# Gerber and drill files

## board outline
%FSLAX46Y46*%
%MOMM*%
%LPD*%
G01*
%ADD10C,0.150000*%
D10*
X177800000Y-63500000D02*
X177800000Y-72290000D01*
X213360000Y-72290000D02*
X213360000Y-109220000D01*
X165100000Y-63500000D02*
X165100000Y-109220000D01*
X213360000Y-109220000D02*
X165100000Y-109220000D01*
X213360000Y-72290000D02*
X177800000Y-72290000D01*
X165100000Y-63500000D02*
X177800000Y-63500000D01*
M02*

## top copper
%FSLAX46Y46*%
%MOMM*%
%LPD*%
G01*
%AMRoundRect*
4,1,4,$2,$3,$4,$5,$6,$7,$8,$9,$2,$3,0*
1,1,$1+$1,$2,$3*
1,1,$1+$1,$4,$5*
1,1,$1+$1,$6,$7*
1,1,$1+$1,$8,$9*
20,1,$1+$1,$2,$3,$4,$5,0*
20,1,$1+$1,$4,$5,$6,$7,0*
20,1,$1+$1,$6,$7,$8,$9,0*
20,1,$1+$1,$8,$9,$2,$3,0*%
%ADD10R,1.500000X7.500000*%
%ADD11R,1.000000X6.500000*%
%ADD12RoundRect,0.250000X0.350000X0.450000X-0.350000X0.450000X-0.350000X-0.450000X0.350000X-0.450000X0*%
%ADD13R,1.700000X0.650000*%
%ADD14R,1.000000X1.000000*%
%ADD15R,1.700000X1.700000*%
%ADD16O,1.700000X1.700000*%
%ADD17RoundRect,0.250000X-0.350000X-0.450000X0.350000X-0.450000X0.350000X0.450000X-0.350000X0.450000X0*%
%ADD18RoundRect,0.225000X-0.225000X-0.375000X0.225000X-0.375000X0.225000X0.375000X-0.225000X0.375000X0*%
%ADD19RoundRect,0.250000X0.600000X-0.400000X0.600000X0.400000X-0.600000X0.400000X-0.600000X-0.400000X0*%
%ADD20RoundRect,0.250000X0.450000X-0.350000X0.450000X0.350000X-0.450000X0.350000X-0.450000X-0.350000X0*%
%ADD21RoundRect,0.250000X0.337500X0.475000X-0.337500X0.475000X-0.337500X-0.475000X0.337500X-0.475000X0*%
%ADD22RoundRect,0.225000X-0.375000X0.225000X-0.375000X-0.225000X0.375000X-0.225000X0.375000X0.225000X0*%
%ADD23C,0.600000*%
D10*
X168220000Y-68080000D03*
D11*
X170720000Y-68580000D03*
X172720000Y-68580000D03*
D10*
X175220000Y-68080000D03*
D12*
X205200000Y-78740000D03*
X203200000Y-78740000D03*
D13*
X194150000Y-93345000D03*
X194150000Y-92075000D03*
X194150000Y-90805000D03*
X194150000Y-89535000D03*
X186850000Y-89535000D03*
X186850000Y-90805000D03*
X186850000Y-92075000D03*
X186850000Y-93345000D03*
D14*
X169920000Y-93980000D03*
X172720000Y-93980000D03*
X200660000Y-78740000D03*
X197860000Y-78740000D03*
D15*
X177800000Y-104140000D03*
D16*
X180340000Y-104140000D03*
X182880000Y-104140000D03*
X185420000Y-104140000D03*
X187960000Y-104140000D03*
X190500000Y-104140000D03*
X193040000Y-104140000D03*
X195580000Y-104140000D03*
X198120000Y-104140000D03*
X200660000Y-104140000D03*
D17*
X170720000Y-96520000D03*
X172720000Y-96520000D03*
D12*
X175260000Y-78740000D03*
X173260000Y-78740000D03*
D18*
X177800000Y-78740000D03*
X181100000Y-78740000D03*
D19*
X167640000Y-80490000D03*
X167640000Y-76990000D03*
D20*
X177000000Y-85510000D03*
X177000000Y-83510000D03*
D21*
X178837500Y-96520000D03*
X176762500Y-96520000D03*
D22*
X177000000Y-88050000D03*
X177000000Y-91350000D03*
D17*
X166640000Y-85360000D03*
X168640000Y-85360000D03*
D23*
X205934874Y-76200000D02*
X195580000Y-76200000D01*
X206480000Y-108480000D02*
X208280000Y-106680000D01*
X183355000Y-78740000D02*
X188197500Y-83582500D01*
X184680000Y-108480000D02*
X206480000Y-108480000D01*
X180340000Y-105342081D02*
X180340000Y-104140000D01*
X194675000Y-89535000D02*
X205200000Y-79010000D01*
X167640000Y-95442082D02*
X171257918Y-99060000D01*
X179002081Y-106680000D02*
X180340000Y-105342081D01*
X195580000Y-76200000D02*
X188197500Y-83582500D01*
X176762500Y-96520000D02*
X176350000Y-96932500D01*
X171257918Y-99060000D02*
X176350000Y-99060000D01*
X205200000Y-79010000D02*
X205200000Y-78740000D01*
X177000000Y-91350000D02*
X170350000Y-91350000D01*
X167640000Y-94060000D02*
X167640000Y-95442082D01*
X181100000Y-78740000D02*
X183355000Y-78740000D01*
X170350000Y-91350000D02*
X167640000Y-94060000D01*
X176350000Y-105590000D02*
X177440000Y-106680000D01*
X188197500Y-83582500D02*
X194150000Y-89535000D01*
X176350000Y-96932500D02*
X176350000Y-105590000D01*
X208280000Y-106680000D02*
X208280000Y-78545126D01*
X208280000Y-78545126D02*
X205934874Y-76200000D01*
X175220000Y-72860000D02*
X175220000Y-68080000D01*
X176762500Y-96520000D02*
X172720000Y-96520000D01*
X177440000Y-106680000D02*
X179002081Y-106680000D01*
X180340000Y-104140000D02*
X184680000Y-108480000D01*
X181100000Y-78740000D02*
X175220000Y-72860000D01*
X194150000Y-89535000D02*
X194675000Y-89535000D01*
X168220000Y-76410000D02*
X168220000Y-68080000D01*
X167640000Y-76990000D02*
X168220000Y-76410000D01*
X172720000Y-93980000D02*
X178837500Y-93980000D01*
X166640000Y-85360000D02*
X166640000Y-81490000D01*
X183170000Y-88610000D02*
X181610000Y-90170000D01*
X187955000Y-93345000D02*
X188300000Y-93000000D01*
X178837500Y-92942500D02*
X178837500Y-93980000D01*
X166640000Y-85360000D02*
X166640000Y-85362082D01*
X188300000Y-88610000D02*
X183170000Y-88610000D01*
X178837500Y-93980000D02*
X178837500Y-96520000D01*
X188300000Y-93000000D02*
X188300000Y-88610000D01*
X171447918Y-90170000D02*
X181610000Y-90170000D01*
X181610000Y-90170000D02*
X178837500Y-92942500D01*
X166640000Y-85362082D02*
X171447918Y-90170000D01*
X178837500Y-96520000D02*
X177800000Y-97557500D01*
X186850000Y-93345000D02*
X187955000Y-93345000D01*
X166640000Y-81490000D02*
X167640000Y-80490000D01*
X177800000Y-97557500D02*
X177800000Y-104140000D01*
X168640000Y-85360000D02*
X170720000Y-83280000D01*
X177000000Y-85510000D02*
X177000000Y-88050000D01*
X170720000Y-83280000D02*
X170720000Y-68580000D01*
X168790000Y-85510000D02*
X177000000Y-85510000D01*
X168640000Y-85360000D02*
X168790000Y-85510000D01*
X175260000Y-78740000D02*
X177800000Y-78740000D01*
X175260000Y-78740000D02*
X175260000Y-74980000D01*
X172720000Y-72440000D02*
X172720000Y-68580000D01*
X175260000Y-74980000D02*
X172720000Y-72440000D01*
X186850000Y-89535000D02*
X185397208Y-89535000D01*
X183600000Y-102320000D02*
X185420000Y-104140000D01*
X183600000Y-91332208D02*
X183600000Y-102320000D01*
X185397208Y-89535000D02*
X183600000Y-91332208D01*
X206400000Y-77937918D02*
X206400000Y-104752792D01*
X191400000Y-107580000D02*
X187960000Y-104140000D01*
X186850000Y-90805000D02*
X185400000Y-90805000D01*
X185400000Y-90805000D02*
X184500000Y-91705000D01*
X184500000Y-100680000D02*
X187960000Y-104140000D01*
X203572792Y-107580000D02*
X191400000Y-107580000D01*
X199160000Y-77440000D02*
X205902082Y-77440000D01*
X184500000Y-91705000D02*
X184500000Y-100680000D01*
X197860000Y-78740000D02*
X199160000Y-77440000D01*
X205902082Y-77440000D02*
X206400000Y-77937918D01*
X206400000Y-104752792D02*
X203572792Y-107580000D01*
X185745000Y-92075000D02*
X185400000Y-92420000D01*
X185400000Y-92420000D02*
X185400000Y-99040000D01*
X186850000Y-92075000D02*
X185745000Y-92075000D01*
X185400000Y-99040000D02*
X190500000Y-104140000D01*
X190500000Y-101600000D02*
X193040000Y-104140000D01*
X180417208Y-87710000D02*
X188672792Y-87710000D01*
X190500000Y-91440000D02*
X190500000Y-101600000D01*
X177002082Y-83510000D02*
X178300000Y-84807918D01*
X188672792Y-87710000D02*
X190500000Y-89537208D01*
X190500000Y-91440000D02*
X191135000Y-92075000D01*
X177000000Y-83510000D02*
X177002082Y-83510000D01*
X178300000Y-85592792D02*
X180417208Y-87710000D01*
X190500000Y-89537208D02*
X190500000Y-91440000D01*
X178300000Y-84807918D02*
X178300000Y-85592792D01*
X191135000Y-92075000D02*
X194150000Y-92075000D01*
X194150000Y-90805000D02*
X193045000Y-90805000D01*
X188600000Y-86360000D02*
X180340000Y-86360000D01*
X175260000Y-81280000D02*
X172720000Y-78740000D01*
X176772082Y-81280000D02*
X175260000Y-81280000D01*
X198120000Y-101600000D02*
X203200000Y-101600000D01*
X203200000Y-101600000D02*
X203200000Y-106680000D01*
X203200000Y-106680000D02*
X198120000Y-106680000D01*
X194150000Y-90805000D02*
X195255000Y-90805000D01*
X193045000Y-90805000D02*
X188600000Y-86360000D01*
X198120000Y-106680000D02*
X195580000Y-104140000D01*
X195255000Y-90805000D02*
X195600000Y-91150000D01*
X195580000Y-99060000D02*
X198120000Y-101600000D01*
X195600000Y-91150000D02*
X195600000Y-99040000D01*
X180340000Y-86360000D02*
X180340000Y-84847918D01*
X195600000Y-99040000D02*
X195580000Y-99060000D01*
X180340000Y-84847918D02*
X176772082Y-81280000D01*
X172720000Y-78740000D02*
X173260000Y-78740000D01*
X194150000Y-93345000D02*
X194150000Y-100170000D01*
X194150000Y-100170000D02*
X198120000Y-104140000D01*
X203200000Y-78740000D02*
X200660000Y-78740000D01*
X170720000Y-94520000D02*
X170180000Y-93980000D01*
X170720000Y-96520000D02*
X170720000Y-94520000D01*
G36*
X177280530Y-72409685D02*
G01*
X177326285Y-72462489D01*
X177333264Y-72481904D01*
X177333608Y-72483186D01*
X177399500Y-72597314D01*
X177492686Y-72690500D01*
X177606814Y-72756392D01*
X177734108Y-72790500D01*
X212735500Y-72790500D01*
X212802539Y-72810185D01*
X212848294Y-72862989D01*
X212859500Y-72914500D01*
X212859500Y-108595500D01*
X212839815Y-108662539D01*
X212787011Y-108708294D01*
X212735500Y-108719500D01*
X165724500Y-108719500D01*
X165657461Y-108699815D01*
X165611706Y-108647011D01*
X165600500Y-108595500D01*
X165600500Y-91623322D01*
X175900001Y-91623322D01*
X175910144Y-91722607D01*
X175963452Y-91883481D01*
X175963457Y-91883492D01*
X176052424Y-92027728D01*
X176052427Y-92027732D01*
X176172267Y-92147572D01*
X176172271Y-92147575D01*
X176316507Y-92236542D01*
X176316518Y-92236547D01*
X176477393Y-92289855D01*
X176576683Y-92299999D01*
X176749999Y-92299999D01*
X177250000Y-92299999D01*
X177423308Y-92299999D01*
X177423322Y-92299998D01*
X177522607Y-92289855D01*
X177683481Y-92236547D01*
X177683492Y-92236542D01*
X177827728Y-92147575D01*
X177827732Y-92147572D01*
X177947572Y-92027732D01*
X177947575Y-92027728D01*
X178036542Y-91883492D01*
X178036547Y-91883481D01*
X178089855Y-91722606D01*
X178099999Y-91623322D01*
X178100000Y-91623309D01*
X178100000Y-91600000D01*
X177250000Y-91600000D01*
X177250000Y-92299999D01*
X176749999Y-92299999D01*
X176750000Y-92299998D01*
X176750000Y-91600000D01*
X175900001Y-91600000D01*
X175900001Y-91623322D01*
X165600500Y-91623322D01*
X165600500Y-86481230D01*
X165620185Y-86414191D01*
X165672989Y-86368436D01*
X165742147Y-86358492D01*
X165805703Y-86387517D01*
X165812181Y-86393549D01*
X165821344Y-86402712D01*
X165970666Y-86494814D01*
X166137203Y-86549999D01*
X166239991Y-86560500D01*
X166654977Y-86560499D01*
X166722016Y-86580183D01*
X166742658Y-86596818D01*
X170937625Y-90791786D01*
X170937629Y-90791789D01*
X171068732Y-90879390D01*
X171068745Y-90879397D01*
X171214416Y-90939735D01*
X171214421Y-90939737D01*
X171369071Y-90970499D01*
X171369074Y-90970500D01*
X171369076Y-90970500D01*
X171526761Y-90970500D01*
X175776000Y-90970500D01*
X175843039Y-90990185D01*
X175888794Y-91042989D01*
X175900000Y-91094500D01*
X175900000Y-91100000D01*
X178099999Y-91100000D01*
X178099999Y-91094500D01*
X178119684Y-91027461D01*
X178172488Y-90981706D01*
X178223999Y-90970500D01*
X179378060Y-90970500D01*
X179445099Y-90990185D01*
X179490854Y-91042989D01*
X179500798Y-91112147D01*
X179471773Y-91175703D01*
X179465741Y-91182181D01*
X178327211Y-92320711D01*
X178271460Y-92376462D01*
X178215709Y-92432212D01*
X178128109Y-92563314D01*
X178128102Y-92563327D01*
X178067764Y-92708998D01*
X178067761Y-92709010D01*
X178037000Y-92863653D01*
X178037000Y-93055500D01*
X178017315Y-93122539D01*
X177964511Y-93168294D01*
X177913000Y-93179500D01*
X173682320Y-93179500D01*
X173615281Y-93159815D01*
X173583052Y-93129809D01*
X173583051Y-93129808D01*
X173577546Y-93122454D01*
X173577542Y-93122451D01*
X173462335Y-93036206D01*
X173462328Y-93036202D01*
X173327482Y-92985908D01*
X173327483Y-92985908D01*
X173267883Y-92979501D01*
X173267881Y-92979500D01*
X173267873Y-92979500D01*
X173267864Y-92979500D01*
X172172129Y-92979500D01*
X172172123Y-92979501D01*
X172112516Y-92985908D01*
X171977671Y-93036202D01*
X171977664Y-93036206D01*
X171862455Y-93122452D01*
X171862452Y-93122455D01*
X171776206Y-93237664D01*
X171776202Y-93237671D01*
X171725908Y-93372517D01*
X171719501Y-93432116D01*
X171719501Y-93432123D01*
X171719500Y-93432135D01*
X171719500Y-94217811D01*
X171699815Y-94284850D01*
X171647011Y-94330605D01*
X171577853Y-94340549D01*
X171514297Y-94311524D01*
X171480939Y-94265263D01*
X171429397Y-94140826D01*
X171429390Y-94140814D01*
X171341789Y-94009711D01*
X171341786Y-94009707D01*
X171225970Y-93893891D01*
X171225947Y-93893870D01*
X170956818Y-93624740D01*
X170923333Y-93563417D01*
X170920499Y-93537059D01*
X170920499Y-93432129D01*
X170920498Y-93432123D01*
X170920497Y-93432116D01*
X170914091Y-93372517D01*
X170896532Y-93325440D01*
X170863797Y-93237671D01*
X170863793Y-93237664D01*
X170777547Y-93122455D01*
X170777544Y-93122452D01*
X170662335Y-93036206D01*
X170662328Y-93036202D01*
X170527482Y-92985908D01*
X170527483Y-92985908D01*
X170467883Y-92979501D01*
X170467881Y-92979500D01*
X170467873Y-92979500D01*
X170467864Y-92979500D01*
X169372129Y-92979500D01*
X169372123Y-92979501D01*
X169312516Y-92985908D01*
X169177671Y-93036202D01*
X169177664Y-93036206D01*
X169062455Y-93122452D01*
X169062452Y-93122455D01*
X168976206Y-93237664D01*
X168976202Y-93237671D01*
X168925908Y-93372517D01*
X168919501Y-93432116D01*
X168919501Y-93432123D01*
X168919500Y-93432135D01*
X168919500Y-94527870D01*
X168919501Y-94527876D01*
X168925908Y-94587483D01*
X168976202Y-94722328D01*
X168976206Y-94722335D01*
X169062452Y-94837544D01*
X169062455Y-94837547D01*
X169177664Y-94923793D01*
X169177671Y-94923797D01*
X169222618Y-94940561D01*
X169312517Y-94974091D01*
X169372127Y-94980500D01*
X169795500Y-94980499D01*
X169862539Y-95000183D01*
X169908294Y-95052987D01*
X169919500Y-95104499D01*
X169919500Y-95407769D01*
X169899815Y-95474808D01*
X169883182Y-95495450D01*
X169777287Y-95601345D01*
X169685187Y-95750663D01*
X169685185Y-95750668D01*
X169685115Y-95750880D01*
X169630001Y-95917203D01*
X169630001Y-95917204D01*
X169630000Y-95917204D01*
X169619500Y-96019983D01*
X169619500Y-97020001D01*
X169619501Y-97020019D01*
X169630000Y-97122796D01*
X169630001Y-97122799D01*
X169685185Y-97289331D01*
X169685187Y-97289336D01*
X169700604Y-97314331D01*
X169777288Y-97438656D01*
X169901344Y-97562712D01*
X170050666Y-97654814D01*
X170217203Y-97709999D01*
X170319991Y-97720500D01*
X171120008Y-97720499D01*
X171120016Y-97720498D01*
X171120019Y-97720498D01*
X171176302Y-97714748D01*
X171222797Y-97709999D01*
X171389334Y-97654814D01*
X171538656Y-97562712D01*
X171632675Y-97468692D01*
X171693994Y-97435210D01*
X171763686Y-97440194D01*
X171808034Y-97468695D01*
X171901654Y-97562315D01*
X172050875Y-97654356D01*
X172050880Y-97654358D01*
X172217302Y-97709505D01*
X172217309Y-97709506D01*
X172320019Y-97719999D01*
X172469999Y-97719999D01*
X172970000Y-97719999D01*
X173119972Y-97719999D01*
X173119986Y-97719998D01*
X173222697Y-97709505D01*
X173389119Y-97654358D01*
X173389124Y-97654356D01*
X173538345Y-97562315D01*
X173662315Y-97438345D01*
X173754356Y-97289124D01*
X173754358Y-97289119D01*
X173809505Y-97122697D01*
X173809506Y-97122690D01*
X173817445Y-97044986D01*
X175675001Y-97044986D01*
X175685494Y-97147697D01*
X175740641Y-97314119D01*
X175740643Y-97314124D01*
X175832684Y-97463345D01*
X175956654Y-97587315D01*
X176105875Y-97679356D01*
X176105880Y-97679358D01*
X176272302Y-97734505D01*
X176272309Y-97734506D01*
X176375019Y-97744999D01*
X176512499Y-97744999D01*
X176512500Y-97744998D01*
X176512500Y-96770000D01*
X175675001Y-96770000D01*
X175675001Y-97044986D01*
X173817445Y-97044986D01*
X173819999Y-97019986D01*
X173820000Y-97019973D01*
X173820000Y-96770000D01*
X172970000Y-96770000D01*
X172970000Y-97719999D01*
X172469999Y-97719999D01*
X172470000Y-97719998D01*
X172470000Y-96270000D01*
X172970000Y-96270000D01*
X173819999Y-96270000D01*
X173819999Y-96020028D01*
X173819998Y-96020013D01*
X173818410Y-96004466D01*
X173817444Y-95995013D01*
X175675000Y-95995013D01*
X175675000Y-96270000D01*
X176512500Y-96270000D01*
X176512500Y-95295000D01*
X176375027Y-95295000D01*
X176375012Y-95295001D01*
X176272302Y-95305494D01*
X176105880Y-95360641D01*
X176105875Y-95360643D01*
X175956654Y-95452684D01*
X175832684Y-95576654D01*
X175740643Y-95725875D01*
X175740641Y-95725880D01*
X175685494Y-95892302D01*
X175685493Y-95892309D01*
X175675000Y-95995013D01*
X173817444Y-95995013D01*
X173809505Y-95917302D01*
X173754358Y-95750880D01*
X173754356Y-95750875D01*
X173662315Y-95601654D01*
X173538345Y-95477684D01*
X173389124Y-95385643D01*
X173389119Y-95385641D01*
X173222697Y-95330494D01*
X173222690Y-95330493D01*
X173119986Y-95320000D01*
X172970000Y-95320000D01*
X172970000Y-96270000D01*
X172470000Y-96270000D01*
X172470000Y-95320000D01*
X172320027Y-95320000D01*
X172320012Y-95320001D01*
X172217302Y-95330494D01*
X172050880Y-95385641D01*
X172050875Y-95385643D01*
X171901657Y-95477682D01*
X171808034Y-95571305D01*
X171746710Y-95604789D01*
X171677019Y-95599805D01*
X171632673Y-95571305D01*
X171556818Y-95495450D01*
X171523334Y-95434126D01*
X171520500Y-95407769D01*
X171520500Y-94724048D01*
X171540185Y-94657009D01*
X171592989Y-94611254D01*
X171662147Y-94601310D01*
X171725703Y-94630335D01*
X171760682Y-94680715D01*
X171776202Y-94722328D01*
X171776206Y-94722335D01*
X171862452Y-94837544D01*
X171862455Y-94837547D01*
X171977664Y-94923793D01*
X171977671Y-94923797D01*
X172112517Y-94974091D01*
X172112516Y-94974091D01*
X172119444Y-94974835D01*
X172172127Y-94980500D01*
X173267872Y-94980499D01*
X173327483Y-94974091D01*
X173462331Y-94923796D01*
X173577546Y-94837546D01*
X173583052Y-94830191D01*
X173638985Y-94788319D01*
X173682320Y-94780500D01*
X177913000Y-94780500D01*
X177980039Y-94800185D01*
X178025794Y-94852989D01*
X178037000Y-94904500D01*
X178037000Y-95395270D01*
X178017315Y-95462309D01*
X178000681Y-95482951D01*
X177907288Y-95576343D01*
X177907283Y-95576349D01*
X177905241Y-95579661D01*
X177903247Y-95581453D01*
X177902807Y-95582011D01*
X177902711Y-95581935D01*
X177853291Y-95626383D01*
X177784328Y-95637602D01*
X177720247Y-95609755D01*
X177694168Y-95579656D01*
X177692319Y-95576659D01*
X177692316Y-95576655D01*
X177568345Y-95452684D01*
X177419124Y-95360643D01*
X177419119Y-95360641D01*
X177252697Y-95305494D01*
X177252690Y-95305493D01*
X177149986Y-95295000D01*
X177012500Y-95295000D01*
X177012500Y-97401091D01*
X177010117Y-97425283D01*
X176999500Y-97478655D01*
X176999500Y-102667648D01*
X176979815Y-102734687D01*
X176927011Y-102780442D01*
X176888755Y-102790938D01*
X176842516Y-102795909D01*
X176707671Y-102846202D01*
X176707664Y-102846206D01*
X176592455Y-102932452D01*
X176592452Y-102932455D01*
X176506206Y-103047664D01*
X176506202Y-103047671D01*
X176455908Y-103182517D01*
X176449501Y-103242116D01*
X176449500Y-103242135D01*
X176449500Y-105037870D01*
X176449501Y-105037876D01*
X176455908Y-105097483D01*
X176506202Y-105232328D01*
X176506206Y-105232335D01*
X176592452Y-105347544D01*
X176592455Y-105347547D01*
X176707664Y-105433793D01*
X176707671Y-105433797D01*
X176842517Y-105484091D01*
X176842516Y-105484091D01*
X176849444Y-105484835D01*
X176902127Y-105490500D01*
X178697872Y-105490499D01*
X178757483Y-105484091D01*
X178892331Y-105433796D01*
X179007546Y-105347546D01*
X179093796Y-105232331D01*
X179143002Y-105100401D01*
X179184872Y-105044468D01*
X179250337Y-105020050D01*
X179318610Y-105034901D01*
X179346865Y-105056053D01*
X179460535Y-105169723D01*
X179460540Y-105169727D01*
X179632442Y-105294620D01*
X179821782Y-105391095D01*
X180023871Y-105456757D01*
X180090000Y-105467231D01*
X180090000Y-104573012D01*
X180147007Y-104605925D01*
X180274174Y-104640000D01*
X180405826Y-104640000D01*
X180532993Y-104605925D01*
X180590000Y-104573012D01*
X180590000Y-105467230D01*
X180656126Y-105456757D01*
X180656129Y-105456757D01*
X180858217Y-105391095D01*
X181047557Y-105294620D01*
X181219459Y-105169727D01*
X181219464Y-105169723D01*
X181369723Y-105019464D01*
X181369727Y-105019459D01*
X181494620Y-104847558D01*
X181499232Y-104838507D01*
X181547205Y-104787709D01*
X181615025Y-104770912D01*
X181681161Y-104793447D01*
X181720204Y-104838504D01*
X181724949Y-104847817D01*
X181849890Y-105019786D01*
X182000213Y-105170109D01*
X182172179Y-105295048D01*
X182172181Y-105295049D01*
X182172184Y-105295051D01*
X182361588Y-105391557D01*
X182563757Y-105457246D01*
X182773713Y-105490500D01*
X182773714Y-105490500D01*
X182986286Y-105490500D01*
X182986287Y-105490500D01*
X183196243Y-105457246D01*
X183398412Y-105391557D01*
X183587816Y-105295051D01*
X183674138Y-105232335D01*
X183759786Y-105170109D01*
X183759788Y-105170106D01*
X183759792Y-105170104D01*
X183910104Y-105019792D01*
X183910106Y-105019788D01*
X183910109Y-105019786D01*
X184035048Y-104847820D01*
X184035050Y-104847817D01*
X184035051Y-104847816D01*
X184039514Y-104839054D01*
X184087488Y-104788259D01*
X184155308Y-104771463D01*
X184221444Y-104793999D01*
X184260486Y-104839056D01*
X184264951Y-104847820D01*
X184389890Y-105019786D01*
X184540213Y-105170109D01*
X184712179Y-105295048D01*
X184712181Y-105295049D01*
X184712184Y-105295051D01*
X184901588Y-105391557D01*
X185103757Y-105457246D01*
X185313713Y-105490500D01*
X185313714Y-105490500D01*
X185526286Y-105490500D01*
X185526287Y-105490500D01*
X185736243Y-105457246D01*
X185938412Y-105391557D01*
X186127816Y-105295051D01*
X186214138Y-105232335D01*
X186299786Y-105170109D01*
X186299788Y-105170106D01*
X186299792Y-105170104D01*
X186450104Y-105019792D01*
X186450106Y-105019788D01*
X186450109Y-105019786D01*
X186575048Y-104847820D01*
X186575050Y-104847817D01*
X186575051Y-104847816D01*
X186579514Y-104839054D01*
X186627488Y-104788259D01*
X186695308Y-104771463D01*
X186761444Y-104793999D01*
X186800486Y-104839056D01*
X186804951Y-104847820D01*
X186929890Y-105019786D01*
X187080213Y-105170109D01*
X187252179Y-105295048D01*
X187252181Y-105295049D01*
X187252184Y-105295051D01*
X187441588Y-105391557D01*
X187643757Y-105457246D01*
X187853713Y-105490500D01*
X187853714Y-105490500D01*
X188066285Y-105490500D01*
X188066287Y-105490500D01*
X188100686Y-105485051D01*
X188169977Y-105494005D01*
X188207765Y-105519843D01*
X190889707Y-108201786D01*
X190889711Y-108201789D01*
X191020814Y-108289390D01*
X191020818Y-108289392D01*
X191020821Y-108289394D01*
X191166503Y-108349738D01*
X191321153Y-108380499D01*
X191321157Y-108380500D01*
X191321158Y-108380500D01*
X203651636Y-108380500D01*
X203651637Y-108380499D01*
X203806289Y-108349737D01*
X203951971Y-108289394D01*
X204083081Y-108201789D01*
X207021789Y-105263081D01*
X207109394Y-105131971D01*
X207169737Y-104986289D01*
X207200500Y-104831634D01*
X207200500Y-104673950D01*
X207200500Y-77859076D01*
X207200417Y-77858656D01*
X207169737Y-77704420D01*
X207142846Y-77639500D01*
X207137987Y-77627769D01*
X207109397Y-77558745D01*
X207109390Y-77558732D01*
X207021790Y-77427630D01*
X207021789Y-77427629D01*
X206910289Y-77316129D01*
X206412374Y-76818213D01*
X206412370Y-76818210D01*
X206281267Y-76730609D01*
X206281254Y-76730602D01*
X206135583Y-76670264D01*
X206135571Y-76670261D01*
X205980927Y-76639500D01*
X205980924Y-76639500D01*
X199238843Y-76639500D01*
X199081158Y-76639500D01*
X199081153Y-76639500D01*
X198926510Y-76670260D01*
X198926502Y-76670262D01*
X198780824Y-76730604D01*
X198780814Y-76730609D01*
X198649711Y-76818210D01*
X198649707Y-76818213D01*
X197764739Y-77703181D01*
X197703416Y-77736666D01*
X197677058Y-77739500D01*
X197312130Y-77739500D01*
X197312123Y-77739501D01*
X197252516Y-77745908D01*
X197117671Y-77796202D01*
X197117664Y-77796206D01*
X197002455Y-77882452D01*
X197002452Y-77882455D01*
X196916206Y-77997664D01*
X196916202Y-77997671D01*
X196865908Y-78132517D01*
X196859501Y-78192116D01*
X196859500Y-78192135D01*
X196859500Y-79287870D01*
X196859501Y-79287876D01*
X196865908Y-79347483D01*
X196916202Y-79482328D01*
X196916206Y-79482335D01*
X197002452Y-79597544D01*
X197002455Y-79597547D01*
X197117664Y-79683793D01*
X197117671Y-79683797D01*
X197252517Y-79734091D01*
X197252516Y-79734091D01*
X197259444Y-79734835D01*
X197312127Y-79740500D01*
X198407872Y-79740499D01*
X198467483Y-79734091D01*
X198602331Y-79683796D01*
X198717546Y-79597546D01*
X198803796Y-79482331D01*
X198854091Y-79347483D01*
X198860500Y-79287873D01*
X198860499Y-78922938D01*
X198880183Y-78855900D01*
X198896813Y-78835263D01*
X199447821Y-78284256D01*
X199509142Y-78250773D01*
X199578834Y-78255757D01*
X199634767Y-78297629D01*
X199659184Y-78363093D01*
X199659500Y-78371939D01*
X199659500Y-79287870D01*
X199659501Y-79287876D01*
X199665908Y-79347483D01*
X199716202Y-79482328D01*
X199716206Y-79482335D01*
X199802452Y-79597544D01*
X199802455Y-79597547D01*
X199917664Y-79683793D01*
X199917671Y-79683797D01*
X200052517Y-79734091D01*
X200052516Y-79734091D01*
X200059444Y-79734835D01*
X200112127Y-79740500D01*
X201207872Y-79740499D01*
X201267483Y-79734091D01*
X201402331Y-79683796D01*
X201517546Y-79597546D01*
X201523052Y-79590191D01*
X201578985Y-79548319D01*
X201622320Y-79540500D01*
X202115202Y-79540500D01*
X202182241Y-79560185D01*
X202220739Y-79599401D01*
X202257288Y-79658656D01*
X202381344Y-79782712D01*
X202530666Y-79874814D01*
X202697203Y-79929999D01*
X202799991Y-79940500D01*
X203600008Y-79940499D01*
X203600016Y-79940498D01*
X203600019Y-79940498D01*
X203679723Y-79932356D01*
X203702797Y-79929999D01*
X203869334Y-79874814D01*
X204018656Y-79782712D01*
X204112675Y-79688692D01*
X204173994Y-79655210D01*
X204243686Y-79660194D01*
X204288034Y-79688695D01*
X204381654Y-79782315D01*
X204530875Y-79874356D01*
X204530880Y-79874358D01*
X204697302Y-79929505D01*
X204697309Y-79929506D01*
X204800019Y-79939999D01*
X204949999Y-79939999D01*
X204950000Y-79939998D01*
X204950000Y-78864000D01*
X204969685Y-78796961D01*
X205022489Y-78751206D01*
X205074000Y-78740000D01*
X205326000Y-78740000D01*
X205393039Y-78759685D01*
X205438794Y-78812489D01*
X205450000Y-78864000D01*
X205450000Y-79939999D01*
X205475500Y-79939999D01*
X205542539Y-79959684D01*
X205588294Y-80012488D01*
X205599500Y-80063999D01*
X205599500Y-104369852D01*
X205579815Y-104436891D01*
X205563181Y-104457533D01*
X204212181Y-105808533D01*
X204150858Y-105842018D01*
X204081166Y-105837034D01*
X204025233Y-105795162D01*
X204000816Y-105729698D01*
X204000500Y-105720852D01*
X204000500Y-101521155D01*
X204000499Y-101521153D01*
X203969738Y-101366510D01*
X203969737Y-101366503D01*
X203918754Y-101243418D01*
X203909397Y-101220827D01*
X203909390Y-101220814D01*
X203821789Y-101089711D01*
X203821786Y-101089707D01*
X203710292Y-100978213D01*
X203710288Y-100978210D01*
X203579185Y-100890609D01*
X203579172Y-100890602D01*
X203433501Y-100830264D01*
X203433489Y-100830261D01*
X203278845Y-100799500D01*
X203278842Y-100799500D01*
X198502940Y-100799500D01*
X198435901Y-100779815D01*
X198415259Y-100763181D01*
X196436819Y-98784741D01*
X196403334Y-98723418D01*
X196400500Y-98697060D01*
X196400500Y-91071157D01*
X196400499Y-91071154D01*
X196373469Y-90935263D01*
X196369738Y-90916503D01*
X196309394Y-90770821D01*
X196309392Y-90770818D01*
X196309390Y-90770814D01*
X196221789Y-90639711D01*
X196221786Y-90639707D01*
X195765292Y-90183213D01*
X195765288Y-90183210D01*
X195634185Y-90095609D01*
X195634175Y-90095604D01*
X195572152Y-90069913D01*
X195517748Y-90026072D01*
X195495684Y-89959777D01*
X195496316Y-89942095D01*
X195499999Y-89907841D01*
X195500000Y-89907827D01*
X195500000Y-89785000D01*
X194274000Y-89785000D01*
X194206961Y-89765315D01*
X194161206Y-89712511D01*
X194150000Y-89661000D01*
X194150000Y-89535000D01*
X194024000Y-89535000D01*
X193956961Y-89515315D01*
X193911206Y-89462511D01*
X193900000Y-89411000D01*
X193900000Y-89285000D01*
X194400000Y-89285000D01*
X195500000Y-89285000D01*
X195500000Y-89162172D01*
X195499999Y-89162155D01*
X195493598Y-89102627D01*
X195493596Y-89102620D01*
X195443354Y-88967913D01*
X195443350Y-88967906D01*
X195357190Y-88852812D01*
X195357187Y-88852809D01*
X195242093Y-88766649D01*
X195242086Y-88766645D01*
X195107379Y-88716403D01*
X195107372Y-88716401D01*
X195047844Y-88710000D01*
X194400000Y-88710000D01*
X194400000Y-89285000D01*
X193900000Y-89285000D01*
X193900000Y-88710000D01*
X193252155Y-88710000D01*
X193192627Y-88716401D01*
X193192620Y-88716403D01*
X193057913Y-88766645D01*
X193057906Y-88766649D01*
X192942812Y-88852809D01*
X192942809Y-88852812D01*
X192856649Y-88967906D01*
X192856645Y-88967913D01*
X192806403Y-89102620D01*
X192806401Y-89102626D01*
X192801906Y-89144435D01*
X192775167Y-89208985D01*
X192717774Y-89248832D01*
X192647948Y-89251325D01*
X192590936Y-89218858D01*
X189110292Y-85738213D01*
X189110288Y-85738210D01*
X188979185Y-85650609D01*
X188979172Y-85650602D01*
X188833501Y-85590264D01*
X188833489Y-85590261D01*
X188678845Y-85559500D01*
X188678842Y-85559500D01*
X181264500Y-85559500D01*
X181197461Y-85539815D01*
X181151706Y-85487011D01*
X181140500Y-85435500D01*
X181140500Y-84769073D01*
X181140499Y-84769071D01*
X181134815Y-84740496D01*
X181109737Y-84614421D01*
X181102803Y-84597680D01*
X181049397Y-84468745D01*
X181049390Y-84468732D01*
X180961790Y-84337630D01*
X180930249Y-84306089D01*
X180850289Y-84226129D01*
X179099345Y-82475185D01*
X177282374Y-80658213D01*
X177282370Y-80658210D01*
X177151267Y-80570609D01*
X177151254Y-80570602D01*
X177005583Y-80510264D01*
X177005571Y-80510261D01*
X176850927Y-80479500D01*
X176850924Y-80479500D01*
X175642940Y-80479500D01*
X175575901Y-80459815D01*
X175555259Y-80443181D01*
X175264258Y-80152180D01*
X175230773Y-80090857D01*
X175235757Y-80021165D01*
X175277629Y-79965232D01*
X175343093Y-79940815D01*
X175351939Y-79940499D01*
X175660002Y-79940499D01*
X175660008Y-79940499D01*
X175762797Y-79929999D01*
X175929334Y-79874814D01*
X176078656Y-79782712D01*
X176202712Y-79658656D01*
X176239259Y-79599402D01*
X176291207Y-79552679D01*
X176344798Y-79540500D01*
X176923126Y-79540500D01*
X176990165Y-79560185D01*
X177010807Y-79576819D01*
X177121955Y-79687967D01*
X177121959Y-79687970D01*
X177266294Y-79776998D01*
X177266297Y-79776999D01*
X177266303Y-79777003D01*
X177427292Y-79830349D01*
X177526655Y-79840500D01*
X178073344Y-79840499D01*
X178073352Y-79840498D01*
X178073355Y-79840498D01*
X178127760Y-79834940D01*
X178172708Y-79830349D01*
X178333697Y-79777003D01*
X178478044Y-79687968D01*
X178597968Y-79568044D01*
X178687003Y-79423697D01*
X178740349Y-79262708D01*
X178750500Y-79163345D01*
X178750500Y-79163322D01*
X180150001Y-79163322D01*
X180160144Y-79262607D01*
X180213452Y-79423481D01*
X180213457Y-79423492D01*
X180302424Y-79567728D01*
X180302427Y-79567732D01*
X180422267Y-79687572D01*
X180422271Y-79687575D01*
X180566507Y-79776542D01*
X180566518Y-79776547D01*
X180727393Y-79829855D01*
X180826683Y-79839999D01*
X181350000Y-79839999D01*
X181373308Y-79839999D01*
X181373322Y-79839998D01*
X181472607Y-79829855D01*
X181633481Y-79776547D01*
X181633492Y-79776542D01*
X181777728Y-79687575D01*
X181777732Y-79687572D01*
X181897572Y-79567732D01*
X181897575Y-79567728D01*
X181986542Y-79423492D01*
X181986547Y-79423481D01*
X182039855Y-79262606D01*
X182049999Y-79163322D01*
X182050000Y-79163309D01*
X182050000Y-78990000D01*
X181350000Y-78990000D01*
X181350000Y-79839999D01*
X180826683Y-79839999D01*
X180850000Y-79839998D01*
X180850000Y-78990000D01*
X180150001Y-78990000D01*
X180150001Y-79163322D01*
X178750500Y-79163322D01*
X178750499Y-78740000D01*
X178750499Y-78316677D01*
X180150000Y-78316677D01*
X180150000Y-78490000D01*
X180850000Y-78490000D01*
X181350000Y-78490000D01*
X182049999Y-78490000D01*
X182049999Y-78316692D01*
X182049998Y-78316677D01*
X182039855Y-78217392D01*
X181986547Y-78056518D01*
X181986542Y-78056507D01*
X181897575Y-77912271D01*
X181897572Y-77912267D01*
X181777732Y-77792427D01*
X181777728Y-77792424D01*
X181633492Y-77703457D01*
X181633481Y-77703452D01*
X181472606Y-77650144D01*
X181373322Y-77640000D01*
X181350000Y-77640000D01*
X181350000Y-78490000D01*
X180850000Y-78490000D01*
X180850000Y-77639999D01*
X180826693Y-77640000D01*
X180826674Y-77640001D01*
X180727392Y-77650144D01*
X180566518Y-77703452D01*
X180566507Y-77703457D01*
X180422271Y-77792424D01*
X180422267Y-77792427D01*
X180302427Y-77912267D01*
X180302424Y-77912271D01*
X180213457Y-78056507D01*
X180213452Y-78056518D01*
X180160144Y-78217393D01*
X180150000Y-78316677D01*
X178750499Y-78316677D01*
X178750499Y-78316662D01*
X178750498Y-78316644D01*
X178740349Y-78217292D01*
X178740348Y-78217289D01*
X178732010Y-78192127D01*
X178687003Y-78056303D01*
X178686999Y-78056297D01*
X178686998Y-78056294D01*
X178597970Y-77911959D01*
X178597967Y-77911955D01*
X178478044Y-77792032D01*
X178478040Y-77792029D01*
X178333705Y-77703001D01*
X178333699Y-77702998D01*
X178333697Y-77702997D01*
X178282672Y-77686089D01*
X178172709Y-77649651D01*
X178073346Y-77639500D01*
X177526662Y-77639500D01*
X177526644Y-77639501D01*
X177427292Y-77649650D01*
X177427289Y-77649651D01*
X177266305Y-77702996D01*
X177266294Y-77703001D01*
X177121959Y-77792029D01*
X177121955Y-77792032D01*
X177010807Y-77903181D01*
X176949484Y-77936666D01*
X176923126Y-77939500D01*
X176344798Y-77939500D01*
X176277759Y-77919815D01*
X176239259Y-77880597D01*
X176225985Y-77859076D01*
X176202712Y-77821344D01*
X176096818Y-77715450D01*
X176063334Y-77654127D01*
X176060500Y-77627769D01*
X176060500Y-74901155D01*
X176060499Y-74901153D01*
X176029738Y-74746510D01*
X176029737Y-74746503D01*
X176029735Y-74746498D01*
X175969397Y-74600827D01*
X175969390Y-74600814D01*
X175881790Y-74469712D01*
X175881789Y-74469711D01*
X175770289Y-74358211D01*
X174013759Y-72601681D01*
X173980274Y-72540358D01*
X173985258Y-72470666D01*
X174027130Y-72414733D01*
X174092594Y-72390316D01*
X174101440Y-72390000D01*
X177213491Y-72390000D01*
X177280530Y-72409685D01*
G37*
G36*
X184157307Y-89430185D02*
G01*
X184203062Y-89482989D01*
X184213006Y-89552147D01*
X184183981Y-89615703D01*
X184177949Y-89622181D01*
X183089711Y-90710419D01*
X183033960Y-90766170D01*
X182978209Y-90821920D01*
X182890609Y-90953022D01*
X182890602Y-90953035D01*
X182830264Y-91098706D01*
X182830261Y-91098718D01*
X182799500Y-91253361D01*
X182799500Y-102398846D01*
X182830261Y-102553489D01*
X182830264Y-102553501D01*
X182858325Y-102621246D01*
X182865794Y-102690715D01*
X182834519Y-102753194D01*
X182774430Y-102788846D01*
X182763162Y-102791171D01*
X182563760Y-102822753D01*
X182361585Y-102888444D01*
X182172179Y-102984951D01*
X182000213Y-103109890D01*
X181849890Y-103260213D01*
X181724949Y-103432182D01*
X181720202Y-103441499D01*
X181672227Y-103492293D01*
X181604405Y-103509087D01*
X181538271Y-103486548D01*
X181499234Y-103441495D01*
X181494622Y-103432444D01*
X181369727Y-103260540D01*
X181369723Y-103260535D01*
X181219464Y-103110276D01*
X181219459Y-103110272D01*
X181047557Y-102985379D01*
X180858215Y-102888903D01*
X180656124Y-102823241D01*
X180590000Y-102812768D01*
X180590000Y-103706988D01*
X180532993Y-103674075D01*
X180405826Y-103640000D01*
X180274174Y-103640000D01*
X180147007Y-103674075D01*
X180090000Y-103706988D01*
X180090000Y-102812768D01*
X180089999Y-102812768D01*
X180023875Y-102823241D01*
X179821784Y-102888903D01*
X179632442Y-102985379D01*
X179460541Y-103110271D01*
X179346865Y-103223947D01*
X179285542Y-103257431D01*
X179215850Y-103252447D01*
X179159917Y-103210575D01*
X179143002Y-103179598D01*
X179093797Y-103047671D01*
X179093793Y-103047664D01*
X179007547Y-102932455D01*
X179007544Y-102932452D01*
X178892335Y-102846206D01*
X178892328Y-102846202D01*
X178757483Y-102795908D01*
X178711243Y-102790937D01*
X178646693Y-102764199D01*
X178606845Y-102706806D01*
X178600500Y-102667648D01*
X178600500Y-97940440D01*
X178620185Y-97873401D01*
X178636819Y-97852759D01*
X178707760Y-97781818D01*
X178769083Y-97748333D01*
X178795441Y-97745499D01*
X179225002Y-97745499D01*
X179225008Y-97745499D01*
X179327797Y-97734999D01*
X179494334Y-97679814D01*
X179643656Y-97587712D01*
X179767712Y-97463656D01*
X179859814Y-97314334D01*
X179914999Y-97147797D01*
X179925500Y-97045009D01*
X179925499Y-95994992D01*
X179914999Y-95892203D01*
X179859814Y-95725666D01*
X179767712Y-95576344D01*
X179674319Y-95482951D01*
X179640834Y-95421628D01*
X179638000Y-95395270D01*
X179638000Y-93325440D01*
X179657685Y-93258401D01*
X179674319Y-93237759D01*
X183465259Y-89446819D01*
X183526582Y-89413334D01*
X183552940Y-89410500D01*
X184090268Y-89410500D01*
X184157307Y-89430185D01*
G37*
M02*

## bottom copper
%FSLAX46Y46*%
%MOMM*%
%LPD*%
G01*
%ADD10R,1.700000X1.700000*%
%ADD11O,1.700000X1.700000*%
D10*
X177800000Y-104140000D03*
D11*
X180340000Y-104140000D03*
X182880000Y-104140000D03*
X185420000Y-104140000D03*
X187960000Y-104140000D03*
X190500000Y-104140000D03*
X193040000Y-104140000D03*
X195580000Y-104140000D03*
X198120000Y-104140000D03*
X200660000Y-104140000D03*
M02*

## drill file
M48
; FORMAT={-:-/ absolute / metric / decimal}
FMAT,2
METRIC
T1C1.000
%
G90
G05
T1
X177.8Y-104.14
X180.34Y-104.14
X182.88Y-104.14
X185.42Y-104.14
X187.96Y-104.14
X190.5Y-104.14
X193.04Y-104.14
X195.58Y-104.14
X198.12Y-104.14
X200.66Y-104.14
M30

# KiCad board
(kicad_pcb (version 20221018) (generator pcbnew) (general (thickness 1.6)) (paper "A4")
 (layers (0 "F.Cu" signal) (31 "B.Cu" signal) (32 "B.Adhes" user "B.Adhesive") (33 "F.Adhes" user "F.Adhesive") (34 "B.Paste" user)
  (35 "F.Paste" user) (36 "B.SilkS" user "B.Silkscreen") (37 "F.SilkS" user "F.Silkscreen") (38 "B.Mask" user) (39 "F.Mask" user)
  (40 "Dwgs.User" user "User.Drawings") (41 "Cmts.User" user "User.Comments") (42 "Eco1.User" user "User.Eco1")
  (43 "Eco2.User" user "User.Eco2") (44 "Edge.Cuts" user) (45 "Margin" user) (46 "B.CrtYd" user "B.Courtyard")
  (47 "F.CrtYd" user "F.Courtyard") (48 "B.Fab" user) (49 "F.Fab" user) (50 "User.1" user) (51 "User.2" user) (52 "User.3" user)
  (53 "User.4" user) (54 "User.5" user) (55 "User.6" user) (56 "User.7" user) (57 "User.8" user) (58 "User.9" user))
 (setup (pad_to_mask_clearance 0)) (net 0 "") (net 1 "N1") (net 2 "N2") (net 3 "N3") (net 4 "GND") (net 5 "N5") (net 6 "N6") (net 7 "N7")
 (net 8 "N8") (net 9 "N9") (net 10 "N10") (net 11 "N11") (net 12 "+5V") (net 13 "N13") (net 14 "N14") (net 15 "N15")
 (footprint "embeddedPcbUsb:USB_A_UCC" (layer "F.Cu") (at 171.72 68.28 -90)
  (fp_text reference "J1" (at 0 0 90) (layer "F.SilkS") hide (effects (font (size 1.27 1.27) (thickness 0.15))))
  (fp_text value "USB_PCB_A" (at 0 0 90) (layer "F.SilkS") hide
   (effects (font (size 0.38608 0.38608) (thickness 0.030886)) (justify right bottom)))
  (pad "1" smd rect (at -0.2 3.5 270) (size 7.5 1.5) (layers "F.Cu" "F.Paste" "F.Mask") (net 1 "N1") (solder_mask_margin 0.1016))
  (pad "2" smd rect (at 0.3 1 270) (size 6.5 1) (layers "F.Cu" "F.Paste" "F.Mask") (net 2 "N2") (solder_mask_margin 0.1016))
  (pad "3" smd rect (at 0.3 -1 270) (size 6.5 1) (layers "F.Cu" "F.Paste" "F.Mask") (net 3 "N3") (solder_mask_margin 0.1016))
  (pad "4" smd rect (at -0.2 -3.5 270) (size 7.5 1.5) (layers "F.Cu" "F.Paste" "F.Mask") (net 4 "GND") (solder_mask_margin 0.1016)))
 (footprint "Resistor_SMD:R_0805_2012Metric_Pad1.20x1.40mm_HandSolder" (layer "F.Cu") (at 204.2 78.74 180)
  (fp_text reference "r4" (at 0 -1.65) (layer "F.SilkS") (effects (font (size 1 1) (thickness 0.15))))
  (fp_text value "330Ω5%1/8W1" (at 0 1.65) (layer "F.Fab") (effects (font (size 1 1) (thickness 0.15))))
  (pad "1" smd roundrect (at -1 0 180) (size 1.2 1.4) (layers "F.Cu" "F.Paste" "F.Mask") (roundrect_rratio 0.208333) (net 4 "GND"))
  (pad "2" smd roundrect (at 1 0 180) (size 1.2 1.4) (layers "F.Cu" "F.Paste" "F.Mask") (roundrect_rratio 0.208333) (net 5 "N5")))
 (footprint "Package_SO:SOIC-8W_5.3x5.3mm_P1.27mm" (layer "F.Cu") (at 190.5 91.44 180)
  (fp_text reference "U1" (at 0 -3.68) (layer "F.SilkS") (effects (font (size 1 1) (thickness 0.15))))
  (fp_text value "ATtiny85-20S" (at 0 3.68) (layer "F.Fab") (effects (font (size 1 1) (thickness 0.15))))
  (pad "1" smd rect (at -3.65 -1.905 180) (size 1.7 0.65) (layers "F.Cu" "F.Paste" "F.Mask") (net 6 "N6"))
  (pad "2" smd rect (at -3.65 -0.635 180) (size 1.7 0.65) (layers "F.Cu" "F.Paste" "F.Mask") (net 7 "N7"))
  (pad "3" smd rect (at -3.65 0.635 180) (size 1.7 0.65) (layers "F.Cu" "F.Paste" "F.Mask") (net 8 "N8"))
  (pad "4" smd rect (at -3.65 1.905 180) (size 1.7 0.65) (layers "F.Cu" "F.Paste" "F.Mask") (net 4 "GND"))
  (pad "5" smd rect (at 3.65 1.905 180) (size 1.7 0.65) (layers "F.Cu" "F.Paste" "F.Mask") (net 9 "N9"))
  (pad "6" smd rect (at 3.65 0.635 180) (size 1.7 0.65) (layers "F.Cu" "F.Paste" "F.Mask") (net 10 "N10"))
  (pad "7" smd rect (at 3.65 -0.635 180) (size 1.7 0.65) (layers "F.Cu" "F.Paste" "F.Mask") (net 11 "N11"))
  (pad "8" smd rect (at 3.65 -1.905 180) (size 1.7 0.65) (layers "F.Cu" "F.Paste" "F.Mask") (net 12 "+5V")))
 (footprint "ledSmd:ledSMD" (layer "F.Cu") (at 171.72 93.98)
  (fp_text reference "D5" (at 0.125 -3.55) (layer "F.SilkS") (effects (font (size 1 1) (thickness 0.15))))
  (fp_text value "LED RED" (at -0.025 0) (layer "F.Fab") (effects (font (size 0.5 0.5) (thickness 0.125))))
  (pad "1" smd rect (at -1.8 0) (size 1 1) (layers "F.Cu" "F.Paste" "F.Mask") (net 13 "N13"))
  (pad "2" smd rect (at 1 0) (size 1 1) (layers "F.Cu" "F.Paste" "F.Mask") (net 12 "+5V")))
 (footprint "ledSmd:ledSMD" (layer "F.Cu") (at 198.86 78.74 180)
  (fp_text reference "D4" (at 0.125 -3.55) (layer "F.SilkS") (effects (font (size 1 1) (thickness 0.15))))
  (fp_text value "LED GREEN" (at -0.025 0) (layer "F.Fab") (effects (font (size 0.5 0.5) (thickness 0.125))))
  (pad "1" smd rect (at -1.8 0 180) (size 1 1) (layers "F.Cu" "F.Paste" "F.Mask") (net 5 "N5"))
  (pad "2" smd rect (at 1 0 180) (size 1 1) (layers "F.Cu" "F.Paste" "F.Mask") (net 10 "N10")))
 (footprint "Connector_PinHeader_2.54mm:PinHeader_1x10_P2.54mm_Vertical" (layer "F.Cu") (at 177.8 104.14 90)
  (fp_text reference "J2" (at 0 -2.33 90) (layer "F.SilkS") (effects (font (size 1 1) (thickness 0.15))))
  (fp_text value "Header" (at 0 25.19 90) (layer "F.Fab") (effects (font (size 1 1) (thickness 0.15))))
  (pad "1" thru_hole rect (at 0 0 90) (size 1.7 1.7) (drill 1) (layers "*.Cu" "*.Mask") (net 12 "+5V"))
  (pad "2" thru_hole oval (at 0 2.54 90) (size 1.7 1.7) (drill 1) (layers "*.Cu" "*.Mask") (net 4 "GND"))
  (pad "3" thru_hole oval (at 0 5.08 90) (size 1.7 1.7) (drill 1) (layers "*.Cu" "*.Mask") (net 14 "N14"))
  (pad "4" thru_hole oval (at 0 7.62 90) (size 1.7 1.7) (drill 1) (layers "*.Cu" "*.Mask") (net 9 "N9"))
  (pad "5" thru_hole oval (at 0 10.16 90) (size 1.7 1.7) (drill 1) (layers "*.Cu" "*.Mask") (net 10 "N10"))
  (pad "6" thru_hole oval (at 0 12.7 90) (size 1.7 1.7) (drill 1) (layers "*.Cu" "*.Mask") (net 11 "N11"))
  (pad "7" thru_hole oval (at 0 15.24 90) (size 1.7 1.7) (drill 1) (layers "*.Cu" "*.Mask") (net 7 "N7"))
  (pad "8" thru_hole oval (at 0 17.78 90) (size 1.7 1.7) (drill 1) (layers "*.Cu" "*.Mask") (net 8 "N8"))
  (pad "9" thru_hole oval (at 0 20.32 90) (size 1.7 1.7) (drill 1) (layers "*.Cu" "*.Mask") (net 6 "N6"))
  (pad "10" thru_hole oval (at 0 22.86 90) (size 1.7 1.7) (drill 1) (layers "*.Cu" "*.Mask") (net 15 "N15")))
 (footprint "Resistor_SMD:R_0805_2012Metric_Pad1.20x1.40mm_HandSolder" (layer "F.Cu") (at 171.72 96.52)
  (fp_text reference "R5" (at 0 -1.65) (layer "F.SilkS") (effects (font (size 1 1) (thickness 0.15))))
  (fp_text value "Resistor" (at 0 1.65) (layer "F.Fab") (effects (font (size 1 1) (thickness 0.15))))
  (pad "1" smd roundrect (at -1 0) (size 1.2 1.4) (layers "F.Cu" "F.Paste" "F.Mask") (roundrect_rratio 0.208333) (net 13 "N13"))
  (pad "2" smd roundrect (at 1 0) (size 1.2 1.4) (layers "F.Cu" "F.Paste" "F.Mask") (roundrect_rratio 0.208333) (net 4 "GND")))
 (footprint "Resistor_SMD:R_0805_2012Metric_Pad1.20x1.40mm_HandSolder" (layer "F.Cu") (at 174.26 78.74 180)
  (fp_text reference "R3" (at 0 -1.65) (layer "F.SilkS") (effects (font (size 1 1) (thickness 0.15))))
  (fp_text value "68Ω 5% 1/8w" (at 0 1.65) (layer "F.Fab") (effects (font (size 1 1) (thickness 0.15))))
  (pad "1" smd roundrect (at -1 0 180) (size 1.2 1.4) (layers "F.Cu" "F.Paste" "F.Mask") (roundrect_rratio 0.208333) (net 3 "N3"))
  (pad "2" smd roundrect (at 1 0 180) (size 1.2 1.4) (layers "F.Cu" "F.Paste" "F.Mask") (roundrect_rratio 0.208333) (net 8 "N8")))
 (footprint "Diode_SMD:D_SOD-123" (layer "F.Cu") (at 179.45 78.74)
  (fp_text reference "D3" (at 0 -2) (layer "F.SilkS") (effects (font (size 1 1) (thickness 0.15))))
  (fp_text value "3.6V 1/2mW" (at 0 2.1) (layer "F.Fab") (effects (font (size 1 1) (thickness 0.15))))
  (pad "1" smd roundrect (at -1.65 0) (size 0.9 1.2) (layers "F.Cu" "F.Paste" "F.Mask") (roundrect_rratio 0.25) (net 3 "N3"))
  (pad "2" smd roundrect (at 1.65 0) (size 0.9 1.2) (layers "F.Cu" "F.Paste" "F.Mask") (roundrect_rratio 0.25) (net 4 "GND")))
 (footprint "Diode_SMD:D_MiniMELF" (layer "F.Cu") (at 167.64 78.74 90)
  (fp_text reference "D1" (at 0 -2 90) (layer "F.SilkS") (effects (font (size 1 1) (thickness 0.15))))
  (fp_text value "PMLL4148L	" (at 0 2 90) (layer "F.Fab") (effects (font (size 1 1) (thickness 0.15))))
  (pad "1" smd roundrect (at -1.75 0 90) (size 1.3 1.7) (layers "F.Cu" "F.Paste" "F.Mask") (roundrect_rratio 0.1923076923) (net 12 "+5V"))
  (pad "2" smd roundrect (at 1.75 0 90) (size 1.3 1.7) (layers "F.Cu" "F.Paste" "F.Mask") (roundrect_rratio 0.1923076923) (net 1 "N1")))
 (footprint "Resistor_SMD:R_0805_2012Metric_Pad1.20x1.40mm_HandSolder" (layer "F.Cu") (at 177 84.51 90)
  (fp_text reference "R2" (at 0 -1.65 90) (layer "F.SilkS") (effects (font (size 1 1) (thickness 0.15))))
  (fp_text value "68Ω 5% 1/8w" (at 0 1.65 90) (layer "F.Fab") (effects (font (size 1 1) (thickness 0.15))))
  (pad "1" smd roundrect (at -1 0 90) (size 1.2 1.4) (layers "F.Cu" "F.Paste" "F.Mask") (roundrect_rratio 0.208333) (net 2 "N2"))
  (pad "2" smd roundrect (at 1 0 90) (size 1.2 1.4) (layers "F.Cu" "F.Paste" "F.Mask") (roundrect_rratio 0.208333) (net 7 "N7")))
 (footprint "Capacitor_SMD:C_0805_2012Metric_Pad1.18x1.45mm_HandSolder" (layer "F.Cu") (at 177.8 96.52 180)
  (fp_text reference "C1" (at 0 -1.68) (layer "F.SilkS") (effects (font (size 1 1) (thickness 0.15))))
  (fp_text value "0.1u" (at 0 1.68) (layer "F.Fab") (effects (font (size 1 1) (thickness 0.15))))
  (pad "1" smd roundrect (at -1.0375 0 180) (size 1.175 1.45) (layers "F.Cu" "F.Paste" "F.Mask") (roundrect_rratio 0.212766) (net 12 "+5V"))
  (pad "2" smd roundrect (at 1.0375 0 180) (size 1.175 1.45) (layers "F.Cu" "F.Paste" "F.Mask") (roundrect_rratio 0.212766) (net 4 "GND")))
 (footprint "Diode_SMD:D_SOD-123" (layer "F.Cu") (at 177 89.7 -90)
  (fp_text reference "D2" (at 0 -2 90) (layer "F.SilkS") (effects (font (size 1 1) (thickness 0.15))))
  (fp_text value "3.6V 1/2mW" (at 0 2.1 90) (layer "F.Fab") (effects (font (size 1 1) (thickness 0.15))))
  (pad "1" smd roundrect (at -1.65 0 270) (size 0.9 1.2) (layers "F.Cu" "F.Paste" "F.Mask") (roundrect_rratio 0.25) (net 2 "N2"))
  (pad "2" smd roundrect (at 1.65 0 270) (size 0.9 1.2) (layers "F.Cu" "F.Paste" "F.Mask") (roundrect_rratio 0.25) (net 4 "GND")))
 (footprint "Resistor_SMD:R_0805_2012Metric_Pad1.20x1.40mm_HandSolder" (layer "F.Cu") (at 167.64 85.36)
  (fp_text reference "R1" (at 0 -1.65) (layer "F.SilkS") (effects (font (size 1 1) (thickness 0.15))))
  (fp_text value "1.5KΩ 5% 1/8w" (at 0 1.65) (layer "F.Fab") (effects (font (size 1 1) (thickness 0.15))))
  (pad "1" smd roundrect (at -1 0) (size 1.2 1.4) (layers "F.Cu" "F.Paste" "F.Mask") (roundrect_rratio 0.208333) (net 12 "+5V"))
  (pad "2" smd roundrect (at 1 0) (size 1.2 1.4) (layers "F.Cu" "F.Paste" "F.Mask") (roundrect_rratio 0.208333) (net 2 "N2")))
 (gr_line (start 177.8 63.5) (end 177.8 72.29) (stroke (width 0.15) (type default)) (layer "Edge.Cuts"))
 (gr_line (start 213.36 72.29) (end 213.36 109.22) (stroke (width 0.15) (type default)) (layer "Edge.Cuts"))
 (gr_line (start 165.1 63.5) (end 165.1 109.22) (stroke (width 0.15) (type default)) (layer "Edge.Cuts"))
 (gr_line (start 213.36 109.22) (end 165.1 109.22) (stroke (width 0.15) (type default)) (layer "Edge.Cuts"))
 (gr_line (start 213.36 72.29) (end 177.8 72.29) (stroke (width 0.15) (type default)) (layer "Edge.Cuts"))
 (gr_line (start 165.1 63.5) (end 177.8 63.5) (stroke (width 0.15) (type default)) (layer "Edge.Cuts"))
 (segment (start 205.934874 76.2) (end 195.58 76.2) (width 0.6) (layer "F.Cu") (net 4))
 (segment (start 206.48 108.48) (end 208.28 106.68) (width 0.6) (layer "F.Cu") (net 4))
 (segment (start 183.355 78.74) (end 188.1975 83.5825) (width 0.6) (layer "F.Cu") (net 4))
 (segment (start 184.68 108.48) (end 206.48 108.48) (width 0.6) (layer "F.Cu") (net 4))
 (segment (start 180.34 105.342081) (end 180.34 104.14) (width 0.6) (layer "F.Cu") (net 4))
 (segment (start 194.675 89.535) (end 205.2 79.01) (width 0.6) (layer "F.Cu") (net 4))
 (segment (start 167.64 95.442082) (end 171.257918 99.06) (width 0.6) (layer "F.Cu") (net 4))
 (segment (start 179.002081 106.68) (end 180.34 105.342081) (width 0.6) (layer "F.Cu") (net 4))
 (segment (start 195.58 76.2) (end 188.1975 83.5825) (width 0.6) (layer "F.Cu") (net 4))
 (segment (start 176.7625 96.52) (end 176.35 96.9325) (width 0.6) (layer "F.Cu") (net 4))
 (segment (start 171.257918 99.06) (end 176.35 99.06) (width 0.6) (layer "F.Cu") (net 4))
 (segment (start 205.2 79.01) (end 205.2 78.74) (width 0.6) (layer "F.Cu") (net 4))
 (segment (start 177 91.35) (end 170.35 91.35) (width 0.6) (layer "F.Cu") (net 4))
 (segment (start 167.64 94.06) (end 167.64 95.442082) (width 0.6) (layer "F.Cu") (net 4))
 (segment (start 181.1 78.74) (end 183.355 78.74) (width 0.6) (layer "F.Cu") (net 4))
 (segment (start 170.35 91.35) (end 167.64 94.06) (width 0.6) (layer "F.Cu") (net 4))
 (segment (start 176.35 105.59) (end 177.44 106.68) (width 0.6) (layer "F.Cu") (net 4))
 (segment (start 188.1975 83.5825) (end 194.15 89.535) (width 0.6) (layer "F.Cu") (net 4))
 (segment (start 176.35 96.9325) (end 176.35 105.59) (width 0.6) (layer "F.Cu") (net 4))
 (segment (start 208.28 106.68) (end 208.28 78.545126) (width 0.6) (layer "F.Cu") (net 4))
 (segment (start 208.28 78.545126) (end 205.934874 76.2) (width 0.6) (layer "F.Cu") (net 4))
 (segment (start 175.22 72.86) (end 175.22 68.08) (width 0.6) (layer "F.Cu") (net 4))
 (segment (start 176.7625 96.52) (end 172.72 96.52) (width 0.6) (layer "F.Cu") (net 4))
 (segment (start 177.44 106.68) (end 179.002081 106.68) (width 0.6) (layer "F.Cu") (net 4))
 (segment (start 180.34 104.14) (end 184.68 108.48) (width 0.6) (layer "F.Cu") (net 4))
 (segment (start 181.1 78.74) (end 175.22 72.86) (width 0.6) (layer "F.Cu") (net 4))
 (segment (start 194.15 89.535) (end 194.675 89.535) (width 0.6) (layer "F.Cu") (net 4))
 (segment (start 168.22 76.41) (end 168.22 68.08) (width 0.6) (layer "F.Cu") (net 1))
 (segment (start 167.64 76.99) (end 168.22 76.41) (width 0.6) (layer "F.Cu") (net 1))
 (segment (start 172.72 93.98) (end 178.8375 93.98) (width 0.6) (layer "F.Cu") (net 12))
 (segment (start 166.64 85.36) (end 166.64 81.49) (width 0.6) (layer "F.Cu") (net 12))
 (segment (start 183.17 88.61) (end 181.61 90.17) (width 0.6) (layer "F.Cu") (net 12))
 (segment (start 187.955 93.345) (end 188.3 93) (width 0.6) (layer "F.Cu") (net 12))
 (segment (start 178.8375 92.9425) (end 178.8375 93.98) (width 0.6) (layer "F.Cu") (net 12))
 (segment (start 166.64 85.36) (end 166.64 85.362082) (width 0.6) (layer "F.Cu") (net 12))
 (segment (start 188.3 88.61) (end 183.17 88.61) (width 0.6) (layer "F.Cu") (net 12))
 (segment (start 178.8375 93.98) (end 178.8375 96.52) (width 0.6) (layer "F.Cu") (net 12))
 (segment (start 188.3 93) (end 188.3 88.61) (width 0.6) (layer "F.Cu") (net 12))
 (segment (start 171.447918 90.17) (end 181.61 90.17) (width 0.6) (layer "F.Cu") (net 12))
 (segment (start 181.61 90.17) (end 178.8375 92.9425) (width 0.6) (layer "F.Cu") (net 12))
 (segment (start 166.64 85.362082) (end 171.447918 90.17) (width 0.6) (layer "F.Cu") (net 12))
 (segment (start 178.8375 96.52) (end 177.8 97.5575) (width 0.6) (layer "F.Cu") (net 12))
 (segment (start 186.85 93.345) (end 187.955 93.345) (width 0.6) (layer "F.Cu") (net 12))
 (segment (start 166.64 81.49) (end 167.64 80.49) (width 0.6) (layer "F.Cu") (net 12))
 (segment (start 177.8 97.5575) (end 177.8 104.14) (width 0.6) (layer "F.Cu") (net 12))
 (segment (start 168.64 85.36) (end 170.72 83.28) (width 0.6) (layer "F.Cu") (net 2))
 (segment (start 177 85.51) (end 177 88.05) (width 0.6) (layer "F.Cu") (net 2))
 (segment (start 170.72 83.28) (end 170.72 68.58) (width 0.6) (layer "F.Cu") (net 2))
 (segment (start 168.79 85.51) (end 177 85.51) (width 0.6) (layer "F.Cu") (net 2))
 (segment (start 168.64 85.36) (end 168.79 85.51) (width 0.6) (layer "F.Cu") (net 2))
 (segment (start 175.26 78.74) (end 177.8 78.74) (width 0.6) (layer "F.Cu") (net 3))
 (segment (start 175.26 78.74) (end 175.26 74.98) (width 0.6) (layer "F.Cu") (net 3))
 (segment (start 172.72 72.44) (end 172.72 68.58) (width 0.6) (layer "F.Cu") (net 3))
 (segment (start 175.26 74.98) (end 172.72 72.44) (width 0.6) (layer "F.Cu") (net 3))
 (segment (start 186.85 89.535) (end 185.397208 89.535) (width 0.6) (layer "F.Cu") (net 9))
 (segment (start 183.6 102.32) (end 185.42 104.14) (width 0.6) (layer "F.Cu") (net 9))
 (segment (start 183.6 91.332208) (end 183.6 102.32) (width 0.6) (layer "F.Cu") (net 9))
 (segment (start 185.397208 89.535) (end 183.6 91.332208) (width 0.6) (layer "F.Cu") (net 9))
 (segment (start 206.4 77.937918) (end 206.4 104.752792) (width 0.6) (layer "F.Cu") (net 10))
 (segment (start 191.4 107.58) (end 187.96 104.14) (width 0.6) (layer "F.Cu") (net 10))
 (segment (start 186.85 90.805) (end 185.4 90.805) (width 0.6) (layer "F.Cu") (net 10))
 (segment (start 185.4 90.805) (end 184.5 91.705) (width 0.6) (layer "F.Cu") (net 10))
 (segment (start 184.5 100.68) (end 187.96 104.14) (width 0.6) (layer "F.Cu") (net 10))
 (segment (start 203.572792 107.58) (end 191.4 107.58) (width 0.6) (layer "F.Cu") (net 10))
 (segment (start 199.16 77.44) (end 205.902082 77.44) (width 0.6) (layer "F.Cu") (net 10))
 (segment (start 184.5 91.705) (end 184.5 100.68) (width 0.6) (layer "F.Cu") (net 10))
 (segment (start 197.86 78.74) (end 199.16 77.44) (width 0.6) (layer "F.Cu") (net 10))
 (segment (start 205.902082 77.44) (end 206.4 77.937918) (width 0.6) (layer "F.Cu") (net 10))
 (segment (start 206.4 104.752792) (end 203.572792 107.58) (width 0.6) (layer "F.Cu") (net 10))
 (segment (start 185.745 92.075) (end 185.4 92.42) (width 0.6) (layer "F.Cu") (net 11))
 (segment (start 185.4 92.42) (end 185.4 99.04) (width 0.6) (layer "F.Cu") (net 11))
 (segment (start 186.85 92.075) (end 185.745 92.075) (width 0.6) (layer "F.Cu") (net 11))
 (segment (start 185.4 99.04) (end 190.5 104.14) (width 0.6) (layer "F.Cu") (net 11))
 (segment (start 190.5 101.6) (end 193.04 104.14) (width 0.6) (layer "F.Cu") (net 7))
 (segment (start 180.417208 87.71) (end 188.672792 87.71) (width 0.6) (layer "F.Cu") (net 7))
 (segment (start 190.5 91.44) (end 190.5 101.6) (width 0.6) (layer "F.Cu") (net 7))
 (segment (start 177.002082 83.51) (end 178.3 84.807918) (width 0.6) (layer "F.Cu") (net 7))
 (segment (start 188.672792 87.71) (end 190.5 89.537208) (width 0.6) (layer "F.Cu") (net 7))
 (segment (start 190.5 91.44) (end 191.135 92.075) (width 0.6) (layer "F.Cu") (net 7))
 (segment (start 177 83.51) (end 177.002082 83.51) (width 0.6) (layer "F.Cu") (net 7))
 (segment (start 178.3 85.592792) (end 180.417208 87.71) (width 0.6) (layer "F.Cu") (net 7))
 (segment (start 190.5 89.537208) (end 190.5 91.44) (width 0.6) (layer "F.Cu") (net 7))
 (segment (start 178.3 84.807918) (end 178.3 85.592792) (width 0.6) (layer "F.Cu") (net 7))
 (segment (start 191.135 92.075) (end 194.15 92.075) (width 0.6) (layer "F.Cu") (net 7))
 (segment (start 194.15 90.805) (end 193.045 90.805) (width 0.6) (layer "F.Cu") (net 8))
 (segment (start 188.6 86.36) (end 180.34 86.36) (width 0.6) (layer "F.Cu") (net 8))
 (segment (start 175.26 81.28) (end 172.72 78.74) (width 0.6) (layer "F.Cu") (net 8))
 (segment (start 176.772082 81.28) (end 175.26 81.28) (width 0.6) (layer "F.Cu") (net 8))
 (segment (start 198.12 101.6) (end 203.2 101.6) (width 0.6) (layer "F.Cu") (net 8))
 (segment (start 203.2 101.6) (end 203.2 106.68) (width 0.6) (layer "F.Cu") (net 8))
 (segment (start 203.2 106.68) (end 198.12 106.68) (width 0.6) (layer "F.Cu") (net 8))
 (segment (start 194.15 90.805) (end 195.255 90.805) (width 0.6) (layer "F.Cu") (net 8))
 (segment (start 193.045 90.805) (end 188.6 86.36) (width 0.6) (layer "F.Cu") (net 8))
 (segment (start 198.12 106.68) (end 195.58 104.14) (width 0.6) (layer "F.Cu") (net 8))
 (segment (start 195.255 90.805) (end 195.6 91.15) (width 0.6) (layer "F.Cu") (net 8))
 (segment (start 195.58 99.06) (end 198.12 101.6) (width 0.6) (layer "F.Cu") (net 8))
 (segment (start 195.6 91.15) (end 195.6 99.04) (width 0.6) (layer "F.Cu") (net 8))
 (segment (start 180.34 86.36) (end 180.34 84.847918) (width 0.6) (layer "F.Cu") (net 8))
 (segment (start 195.6 99.04) (end 195.58 99.06) (width 0.6) (layer "F.Cu") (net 8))
 (segment (start 180.34 84.847918) (end 176.772082 81.28) (width 0.6) (layer "F.Cu") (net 8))
 (segment (start 172.72 78.74) (end 173.26 78.74) (width 0.6) (layer "F.Cu") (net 8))
 (segment (start 194.15 93.345) (end 194.15 100.17) (width 0.6) (layer "F.Cu") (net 6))
 (segment (start 194.15 100.17) (end 198.12 104.14) (width 0.6) (layer "F.Cu") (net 6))
 (segment (start 203.2 78.74) (end 200.66 78.74) (width 0.6) (layer "F.Cu") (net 5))
 (segment (start 170.72 94.52) (end 170.18 93.98) (width 0.6) (layer "F.Cu") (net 13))
 (segment (start 170.72 96.52) (end 170.72 94.52) (width 0.6) (layer "F.Cu") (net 13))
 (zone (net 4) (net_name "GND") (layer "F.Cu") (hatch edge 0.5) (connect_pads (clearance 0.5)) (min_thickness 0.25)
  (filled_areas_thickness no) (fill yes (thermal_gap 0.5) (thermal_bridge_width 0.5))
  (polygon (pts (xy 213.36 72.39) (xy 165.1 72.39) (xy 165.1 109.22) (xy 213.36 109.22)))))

